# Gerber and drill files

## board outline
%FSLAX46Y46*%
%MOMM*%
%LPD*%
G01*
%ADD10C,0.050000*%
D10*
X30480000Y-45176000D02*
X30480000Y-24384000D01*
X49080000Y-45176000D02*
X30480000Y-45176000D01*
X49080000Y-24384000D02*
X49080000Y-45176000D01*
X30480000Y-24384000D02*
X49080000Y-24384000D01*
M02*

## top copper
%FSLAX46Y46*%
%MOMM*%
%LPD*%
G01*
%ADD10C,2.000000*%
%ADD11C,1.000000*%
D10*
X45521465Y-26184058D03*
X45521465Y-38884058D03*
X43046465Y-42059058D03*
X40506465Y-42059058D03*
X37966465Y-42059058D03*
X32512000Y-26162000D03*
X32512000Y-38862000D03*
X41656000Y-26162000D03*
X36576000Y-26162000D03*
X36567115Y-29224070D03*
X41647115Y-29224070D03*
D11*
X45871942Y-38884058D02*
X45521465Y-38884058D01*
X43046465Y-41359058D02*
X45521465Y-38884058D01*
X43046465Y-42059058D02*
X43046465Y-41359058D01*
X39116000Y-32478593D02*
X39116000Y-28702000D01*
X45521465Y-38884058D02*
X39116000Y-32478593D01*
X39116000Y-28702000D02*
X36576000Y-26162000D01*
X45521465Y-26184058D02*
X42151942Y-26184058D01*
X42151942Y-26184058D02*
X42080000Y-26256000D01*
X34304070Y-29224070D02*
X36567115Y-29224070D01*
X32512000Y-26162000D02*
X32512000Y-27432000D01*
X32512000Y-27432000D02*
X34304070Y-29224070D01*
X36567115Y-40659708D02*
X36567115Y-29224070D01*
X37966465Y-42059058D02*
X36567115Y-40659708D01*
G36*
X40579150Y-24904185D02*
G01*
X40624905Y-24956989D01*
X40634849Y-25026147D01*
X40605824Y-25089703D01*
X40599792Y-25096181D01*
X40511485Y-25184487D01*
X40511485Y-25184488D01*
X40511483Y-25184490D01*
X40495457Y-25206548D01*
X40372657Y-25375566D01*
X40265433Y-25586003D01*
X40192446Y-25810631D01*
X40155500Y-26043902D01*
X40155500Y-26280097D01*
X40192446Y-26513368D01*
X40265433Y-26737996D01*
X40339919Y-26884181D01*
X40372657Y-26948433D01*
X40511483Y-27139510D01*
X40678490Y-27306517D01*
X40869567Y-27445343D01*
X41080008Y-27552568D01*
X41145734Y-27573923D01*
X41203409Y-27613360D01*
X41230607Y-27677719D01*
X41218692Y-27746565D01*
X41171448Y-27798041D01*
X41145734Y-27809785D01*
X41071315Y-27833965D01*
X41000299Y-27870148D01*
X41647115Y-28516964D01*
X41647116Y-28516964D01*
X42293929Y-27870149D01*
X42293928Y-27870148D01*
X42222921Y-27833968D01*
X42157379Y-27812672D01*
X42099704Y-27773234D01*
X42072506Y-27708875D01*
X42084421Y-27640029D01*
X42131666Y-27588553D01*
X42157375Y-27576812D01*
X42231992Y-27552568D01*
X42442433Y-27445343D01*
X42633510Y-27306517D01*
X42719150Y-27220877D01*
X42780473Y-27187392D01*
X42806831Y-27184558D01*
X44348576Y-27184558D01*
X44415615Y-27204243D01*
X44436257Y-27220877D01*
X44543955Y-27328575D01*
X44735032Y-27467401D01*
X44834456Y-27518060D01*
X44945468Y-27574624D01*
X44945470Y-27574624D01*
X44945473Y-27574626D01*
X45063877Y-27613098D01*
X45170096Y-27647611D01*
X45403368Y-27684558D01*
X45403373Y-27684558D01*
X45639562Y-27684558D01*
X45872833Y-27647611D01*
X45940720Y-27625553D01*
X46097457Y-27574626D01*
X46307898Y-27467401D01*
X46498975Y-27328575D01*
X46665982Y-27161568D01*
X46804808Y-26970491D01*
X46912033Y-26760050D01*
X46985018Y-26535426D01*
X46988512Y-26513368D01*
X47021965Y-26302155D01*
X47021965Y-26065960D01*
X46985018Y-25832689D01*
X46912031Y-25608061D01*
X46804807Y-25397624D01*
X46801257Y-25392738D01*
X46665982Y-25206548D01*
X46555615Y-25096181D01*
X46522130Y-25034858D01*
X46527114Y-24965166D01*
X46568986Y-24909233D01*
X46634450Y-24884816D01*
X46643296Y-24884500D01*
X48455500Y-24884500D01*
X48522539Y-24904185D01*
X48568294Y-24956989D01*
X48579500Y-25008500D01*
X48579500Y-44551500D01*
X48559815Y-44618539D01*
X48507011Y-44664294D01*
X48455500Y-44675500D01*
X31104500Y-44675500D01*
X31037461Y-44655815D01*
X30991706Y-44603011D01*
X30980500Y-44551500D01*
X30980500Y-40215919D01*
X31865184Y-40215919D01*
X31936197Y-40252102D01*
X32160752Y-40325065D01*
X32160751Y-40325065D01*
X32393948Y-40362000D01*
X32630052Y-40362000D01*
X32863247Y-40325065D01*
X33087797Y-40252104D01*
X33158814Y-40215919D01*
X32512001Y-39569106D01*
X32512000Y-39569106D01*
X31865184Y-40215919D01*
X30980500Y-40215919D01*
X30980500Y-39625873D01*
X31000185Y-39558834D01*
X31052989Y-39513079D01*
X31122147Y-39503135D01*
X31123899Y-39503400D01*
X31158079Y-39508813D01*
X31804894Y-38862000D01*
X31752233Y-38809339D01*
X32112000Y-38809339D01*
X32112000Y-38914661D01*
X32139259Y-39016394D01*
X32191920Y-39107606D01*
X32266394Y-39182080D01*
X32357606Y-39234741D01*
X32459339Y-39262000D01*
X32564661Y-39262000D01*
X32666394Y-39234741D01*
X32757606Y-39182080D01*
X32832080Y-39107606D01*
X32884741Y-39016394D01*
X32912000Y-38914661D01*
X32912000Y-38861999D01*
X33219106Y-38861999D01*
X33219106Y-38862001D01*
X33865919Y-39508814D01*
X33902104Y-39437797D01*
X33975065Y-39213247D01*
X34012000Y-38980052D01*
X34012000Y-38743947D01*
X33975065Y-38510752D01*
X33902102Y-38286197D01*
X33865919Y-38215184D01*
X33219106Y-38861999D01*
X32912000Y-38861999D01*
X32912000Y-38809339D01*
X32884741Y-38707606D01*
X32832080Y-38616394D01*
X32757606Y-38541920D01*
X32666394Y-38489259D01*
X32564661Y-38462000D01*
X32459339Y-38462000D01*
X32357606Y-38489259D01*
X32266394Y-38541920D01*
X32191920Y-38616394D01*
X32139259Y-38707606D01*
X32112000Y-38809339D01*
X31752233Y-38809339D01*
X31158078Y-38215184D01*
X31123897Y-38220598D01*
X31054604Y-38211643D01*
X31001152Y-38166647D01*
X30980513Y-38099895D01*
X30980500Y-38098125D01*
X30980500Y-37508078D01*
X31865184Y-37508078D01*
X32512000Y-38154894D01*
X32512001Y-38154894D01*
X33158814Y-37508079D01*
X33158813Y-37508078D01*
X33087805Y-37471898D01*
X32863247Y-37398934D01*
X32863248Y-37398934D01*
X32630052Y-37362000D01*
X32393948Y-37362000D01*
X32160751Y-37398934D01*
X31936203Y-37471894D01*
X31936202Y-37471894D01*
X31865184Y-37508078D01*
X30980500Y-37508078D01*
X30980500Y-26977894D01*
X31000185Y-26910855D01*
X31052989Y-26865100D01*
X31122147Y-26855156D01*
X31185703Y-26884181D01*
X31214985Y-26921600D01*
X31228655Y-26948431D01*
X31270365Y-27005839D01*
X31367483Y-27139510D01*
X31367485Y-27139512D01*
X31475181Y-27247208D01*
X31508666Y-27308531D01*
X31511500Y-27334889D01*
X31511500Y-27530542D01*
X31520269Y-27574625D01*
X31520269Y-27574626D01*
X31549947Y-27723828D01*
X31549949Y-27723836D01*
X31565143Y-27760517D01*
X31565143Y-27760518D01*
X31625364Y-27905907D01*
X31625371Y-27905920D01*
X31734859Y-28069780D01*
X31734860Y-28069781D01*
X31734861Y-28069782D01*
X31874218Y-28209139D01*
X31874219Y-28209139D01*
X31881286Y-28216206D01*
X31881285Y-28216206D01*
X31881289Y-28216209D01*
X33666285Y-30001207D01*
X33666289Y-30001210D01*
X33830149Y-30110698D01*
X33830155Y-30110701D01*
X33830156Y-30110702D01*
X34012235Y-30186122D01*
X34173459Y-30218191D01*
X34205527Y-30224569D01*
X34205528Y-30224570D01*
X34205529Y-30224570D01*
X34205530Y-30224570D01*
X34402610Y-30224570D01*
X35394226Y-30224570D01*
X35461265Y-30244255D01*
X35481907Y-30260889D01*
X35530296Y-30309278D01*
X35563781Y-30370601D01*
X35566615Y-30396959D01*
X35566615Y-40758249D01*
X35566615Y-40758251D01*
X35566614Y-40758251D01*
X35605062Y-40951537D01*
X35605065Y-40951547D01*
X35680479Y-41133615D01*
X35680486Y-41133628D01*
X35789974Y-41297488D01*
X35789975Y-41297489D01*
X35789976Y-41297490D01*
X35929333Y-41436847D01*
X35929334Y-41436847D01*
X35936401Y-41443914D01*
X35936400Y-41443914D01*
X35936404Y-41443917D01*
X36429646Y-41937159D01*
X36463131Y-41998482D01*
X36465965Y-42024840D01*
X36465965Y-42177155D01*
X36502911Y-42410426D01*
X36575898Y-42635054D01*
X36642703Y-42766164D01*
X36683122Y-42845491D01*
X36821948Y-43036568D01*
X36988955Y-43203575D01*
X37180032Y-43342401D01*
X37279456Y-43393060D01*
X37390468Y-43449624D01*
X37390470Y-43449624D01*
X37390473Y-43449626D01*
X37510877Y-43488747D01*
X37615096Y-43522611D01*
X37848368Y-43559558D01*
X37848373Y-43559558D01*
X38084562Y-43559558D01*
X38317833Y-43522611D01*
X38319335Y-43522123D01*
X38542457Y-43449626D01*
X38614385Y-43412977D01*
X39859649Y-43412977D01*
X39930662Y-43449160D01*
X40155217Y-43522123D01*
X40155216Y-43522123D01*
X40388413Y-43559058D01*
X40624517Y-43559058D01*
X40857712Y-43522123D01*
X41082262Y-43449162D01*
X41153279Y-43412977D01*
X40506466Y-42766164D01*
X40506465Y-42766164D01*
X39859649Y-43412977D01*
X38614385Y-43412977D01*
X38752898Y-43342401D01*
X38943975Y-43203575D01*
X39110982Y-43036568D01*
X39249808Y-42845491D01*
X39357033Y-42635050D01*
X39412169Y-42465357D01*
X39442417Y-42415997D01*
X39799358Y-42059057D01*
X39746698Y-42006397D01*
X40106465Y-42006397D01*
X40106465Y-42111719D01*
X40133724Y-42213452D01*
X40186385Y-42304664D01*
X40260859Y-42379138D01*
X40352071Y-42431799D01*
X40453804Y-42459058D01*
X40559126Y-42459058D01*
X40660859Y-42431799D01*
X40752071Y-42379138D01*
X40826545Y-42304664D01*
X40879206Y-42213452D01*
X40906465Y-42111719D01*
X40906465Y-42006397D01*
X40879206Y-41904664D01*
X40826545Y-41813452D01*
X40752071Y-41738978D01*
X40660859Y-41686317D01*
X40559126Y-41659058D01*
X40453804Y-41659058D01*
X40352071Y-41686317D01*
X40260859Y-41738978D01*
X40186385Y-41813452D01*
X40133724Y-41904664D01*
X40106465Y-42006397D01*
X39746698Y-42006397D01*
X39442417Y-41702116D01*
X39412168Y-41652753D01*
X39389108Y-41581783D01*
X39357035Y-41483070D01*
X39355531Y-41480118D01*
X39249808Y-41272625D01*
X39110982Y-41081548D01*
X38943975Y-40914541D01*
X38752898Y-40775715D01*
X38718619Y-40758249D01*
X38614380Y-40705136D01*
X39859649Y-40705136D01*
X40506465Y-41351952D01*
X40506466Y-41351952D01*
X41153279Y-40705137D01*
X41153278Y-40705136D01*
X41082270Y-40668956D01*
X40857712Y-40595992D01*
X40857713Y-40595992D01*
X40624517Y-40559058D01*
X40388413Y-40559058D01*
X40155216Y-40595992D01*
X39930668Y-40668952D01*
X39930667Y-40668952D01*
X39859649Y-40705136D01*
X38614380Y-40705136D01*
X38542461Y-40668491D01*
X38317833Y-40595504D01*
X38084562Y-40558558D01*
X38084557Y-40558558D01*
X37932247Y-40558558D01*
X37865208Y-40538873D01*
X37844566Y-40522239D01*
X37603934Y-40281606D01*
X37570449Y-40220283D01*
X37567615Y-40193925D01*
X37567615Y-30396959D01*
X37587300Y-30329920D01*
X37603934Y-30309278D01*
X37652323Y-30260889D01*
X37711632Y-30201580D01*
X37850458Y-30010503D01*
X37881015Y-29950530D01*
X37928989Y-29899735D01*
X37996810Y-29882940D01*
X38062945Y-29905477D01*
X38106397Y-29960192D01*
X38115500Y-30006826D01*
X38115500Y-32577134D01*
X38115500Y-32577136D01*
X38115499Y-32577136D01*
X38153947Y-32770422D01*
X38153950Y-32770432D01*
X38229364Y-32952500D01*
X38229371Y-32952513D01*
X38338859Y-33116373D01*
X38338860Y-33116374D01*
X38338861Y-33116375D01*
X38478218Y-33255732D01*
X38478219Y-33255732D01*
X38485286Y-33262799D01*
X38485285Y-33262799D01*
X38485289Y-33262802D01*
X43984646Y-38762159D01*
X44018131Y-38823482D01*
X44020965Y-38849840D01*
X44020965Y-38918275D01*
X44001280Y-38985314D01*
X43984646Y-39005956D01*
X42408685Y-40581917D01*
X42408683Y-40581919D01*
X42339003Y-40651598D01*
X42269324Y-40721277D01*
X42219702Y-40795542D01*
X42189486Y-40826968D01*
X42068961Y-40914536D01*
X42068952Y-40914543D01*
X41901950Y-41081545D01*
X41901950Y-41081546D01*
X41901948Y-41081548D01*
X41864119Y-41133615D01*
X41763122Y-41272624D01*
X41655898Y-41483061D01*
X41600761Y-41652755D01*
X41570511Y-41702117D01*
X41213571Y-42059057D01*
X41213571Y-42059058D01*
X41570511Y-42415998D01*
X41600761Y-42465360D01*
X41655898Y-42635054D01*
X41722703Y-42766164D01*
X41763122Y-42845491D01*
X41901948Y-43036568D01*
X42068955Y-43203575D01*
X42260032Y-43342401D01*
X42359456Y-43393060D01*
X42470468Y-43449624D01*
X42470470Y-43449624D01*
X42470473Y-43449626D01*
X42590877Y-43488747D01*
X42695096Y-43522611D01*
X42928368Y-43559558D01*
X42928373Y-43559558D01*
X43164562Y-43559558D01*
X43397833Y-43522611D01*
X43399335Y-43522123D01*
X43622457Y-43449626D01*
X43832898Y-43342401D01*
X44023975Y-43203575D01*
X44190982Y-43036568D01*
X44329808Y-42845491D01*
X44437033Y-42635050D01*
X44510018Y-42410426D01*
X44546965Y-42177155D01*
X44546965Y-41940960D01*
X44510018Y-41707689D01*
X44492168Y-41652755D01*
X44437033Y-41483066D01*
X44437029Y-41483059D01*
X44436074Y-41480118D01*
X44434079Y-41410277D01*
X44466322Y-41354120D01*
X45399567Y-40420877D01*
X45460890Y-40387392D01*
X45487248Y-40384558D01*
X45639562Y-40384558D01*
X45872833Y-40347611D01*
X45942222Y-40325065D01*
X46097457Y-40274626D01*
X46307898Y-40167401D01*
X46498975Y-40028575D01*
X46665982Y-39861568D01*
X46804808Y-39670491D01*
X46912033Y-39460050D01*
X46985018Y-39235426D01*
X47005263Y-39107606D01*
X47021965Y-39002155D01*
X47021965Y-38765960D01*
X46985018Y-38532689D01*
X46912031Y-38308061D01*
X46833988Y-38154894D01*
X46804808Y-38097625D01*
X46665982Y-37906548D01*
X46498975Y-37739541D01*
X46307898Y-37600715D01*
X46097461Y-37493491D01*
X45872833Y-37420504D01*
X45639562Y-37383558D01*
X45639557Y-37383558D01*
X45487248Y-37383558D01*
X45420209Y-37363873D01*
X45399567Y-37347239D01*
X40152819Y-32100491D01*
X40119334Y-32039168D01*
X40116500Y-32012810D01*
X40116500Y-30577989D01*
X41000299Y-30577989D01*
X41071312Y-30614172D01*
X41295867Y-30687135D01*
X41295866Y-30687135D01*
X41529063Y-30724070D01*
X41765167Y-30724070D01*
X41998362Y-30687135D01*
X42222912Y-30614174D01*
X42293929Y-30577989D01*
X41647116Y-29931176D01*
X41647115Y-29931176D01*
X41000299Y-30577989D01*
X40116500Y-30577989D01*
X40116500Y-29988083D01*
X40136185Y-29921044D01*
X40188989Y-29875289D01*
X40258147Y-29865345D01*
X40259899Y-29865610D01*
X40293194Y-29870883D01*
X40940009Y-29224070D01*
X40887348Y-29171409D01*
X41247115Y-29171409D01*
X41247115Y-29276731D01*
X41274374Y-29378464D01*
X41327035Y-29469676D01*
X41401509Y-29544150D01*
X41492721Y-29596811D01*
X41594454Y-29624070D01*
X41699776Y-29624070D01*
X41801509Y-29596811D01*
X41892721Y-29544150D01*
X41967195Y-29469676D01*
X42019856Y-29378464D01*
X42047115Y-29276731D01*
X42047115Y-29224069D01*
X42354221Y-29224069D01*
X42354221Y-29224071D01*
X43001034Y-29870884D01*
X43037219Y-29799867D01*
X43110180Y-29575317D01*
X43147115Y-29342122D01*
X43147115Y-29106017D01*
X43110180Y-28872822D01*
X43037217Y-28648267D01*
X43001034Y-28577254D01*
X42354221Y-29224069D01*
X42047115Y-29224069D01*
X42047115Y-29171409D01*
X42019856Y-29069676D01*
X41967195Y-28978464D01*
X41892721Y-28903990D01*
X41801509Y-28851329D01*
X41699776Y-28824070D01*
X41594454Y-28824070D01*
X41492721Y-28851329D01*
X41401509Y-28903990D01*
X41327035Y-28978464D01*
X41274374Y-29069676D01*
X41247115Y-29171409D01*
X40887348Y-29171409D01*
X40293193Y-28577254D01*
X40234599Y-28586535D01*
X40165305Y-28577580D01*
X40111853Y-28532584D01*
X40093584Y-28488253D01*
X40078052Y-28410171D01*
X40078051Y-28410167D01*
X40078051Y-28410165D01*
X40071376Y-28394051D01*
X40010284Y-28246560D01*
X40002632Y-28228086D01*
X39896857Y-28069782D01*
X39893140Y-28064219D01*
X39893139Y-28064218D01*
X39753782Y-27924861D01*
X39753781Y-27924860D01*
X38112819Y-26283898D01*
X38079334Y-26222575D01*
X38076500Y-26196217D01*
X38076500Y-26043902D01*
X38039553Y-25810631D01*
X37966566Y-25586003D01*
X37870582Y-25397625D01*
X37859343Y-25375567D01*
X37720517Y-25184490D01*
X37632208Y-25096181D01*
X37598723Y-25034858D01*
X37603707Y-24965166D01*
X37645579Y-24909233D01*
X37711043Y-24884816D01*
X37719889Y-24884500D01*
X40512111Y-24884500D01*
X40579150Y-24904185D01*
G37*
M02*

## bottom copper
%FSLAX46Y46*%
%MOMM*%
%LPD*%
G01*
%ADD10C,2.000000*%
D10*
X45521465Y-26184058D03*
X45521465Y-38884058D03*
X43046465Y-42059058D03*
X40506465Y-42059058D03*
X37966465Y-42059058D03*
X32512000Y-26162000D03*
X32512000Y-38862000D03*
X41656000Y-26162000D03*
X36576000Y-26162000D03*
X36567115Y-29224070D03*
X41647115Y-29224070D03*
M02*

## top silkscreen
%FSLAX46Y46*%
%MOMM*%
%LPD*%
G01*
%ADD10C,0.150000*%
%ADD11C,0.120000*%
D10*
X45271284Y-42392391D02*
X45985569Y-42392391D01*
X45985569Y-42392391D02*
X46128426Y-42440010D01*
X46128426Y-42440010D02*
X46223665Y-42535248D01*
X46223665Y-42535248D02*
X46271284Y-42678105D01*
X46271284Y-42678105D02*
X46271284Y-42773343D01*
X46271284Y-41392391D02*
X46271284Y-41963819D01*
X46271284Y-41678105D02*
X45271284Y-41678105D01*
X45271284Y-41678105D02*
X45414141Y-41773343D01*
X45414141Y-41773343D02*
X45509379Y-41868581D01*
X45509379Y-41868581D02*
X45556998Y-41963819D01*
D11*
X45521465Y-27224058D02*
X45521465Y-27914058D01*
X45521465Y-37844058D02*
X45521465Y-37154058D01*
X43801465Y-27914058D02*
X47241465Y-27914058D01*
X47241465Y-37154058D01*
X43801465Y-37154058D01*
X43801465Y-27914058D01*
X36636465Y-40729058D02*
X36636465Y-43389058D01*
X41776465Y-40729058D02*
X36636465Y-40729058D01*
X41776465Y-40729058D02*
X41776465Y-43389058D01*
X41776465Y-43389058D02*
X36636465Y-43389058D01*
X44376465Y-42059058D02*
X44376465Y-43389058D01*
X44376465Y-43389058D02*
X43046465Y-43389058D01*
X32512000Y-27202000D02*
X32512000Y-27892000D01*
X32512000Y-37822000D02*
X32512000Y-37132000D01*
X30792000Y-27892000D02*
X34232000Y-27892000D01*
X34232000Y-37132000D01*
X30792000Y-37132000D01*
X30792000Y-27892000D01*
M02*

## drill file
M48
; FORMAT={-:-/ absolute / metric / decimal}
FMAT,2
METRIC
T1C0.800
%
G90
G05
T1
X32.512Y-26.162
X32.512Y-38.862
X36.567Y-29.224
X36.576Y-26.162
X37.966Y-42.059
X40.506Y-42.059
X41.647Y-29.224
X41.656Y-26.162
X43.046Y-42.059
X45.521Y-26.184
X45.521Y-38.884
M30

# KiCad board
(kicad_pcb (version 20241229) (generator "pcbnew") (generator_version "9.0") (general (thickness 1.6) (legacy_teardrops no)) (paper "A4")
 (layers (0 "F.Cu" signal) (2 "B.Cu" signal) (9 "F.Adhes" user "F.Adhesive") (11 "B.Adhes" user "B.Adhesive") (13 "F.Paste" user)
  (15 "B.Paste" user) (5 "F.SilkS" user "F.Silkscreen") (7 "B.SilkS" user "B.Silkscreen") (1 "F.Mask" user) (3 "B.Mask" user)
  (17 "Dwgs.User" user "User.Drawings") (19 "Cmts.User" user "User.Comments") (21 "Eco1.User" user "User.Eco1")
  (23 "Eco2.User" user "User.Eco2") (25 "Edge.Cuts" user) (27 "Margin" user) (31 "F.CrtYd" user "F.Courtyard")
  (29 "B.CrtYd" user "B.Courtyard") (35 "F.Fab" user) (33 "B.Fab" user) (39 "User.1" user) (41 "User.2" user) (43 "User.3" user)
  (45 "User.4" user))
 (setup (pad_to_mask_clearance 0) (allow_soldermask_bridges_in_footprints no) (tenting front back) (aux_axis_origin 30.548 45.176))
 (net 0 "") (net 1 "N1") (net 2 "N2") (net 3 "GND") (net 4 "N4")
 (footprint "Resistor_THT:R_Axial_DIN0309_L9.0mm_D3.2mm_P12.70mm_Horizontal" (layer "F.Cu") (at 45.521465 26.184058 -90)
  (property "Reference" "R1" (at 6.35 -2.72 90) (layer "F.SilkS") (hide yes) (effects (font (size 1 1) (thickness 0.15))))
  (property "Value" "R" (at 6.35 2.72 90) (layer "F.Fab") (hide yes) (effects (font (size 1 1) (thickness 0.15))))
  (fp_line (start 1.04 0) (end 1.73 0) (stroke (width 0.12) (type solid)) (layer "F.SilkS"))
  (fp_line (start 11.66 0) (end 10.97 0) (stroke (width 0.12) (type solid)) (layer "F.SilkS"))
  (fp_rect (start 1.73 -1.72) (end 10.97 1.72) (stroke (width 0.12) (type solid)) (fill no) (layer "F.SilkS"))
  (pad "1" thru_hole circle (at 0 0 270) (size 2 2) (drill 0.8) (layers "*.Cu" "*.Mask") (remove_unused_layers no) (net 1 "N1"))
  (pad "2" thru_hole circle (at 12.7 0 270) (size 2 2) (drill 0.8) (layers "*.Cu" "*.Mask") (remove_unused_layers no) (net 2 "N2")))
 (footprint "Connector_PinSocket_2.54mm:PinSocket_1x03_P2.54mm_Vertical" (layer "F.Cu") (at 43.046465 42.059058 -90)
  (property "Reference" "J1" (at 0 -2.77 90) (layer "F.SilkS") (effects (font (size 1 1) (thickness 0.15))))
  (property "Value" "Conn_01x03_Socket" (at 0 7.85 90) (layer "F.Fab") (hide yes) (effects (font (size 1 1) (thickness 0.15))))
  (fp_line (start -1.33 6.41) (end 1.33 6.41) (stroke (width 0.12) (type solid)) (layer "F.SilkS"))
  (fp_line (start -1.33 1.27) (end -1.33 6.41) (stroke (width 0.12) (type solid)) (layer "F.SilkS"))
  (fp_line (start -1.33 1.27) (end 1.33 1.27) (stroke (width 0.12) (type solid)) (layer "F.SilkS"))
  (fp_line (start 1.33 1.27) (end 1.33 6.41) (stroke (width 0.12) (type solid)) (layer "F.SilkS"))
  (fp_line (start 0 -1.33) (end 1.33 -1.33) (stroke (width 0.12) (type solid)) (layer "F.SilkS"))
  (fp_line (start 1.33 -1.33) (end 1.33 0) (stroke (width 0.12) (type solid)) (layer "F.SilkS"))
  (pad "1" thru_hole circle (at 0 0 270) (size 2 2) (drill 0.8) (layers "*.Cu" "*.Mask") (remove_unused_layers no) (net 2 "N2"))
  (pad "2" thru_hole circle (at 0 2.54 270) (size 2 2) (drill 0.8) (layers "*.Cu" "*.Mask") (remove_unused_layers no) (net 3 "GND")
   (thermal_bridge_width 1))
  (pad "3" thru_hole circle (at 0 5.08 270) (size 2 2) (drill 0.8) (layers "*.Cu" "*.Mask") (remove_unused_layers no) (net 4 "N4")))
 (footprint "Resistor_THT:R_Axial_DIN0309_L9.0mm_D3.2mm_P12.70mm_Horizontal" (layer "F.Cu") (at 32.512 26.162 -90)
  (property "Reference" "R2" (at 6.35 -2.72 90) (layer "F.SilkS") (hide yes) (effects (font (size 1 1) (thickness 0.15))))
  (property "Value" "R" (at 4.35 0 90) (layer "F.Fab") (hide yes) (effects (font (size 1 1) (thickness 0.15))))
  (fp_line (start 1.04 0) (end 1.73 0) (stroke (width 0.12) (type solid)) (layer "F.SilkS"))
  (fp_line (start 11.66 0) (end 10.97 0) (stroke (width 0.12) (type solid)) (layer "F.SilkS"))
  (fp_rect (start 1.73 -1.72) (end 10.97 1.72) (stroke (width 0.12) (type solid)) (fill no) (layer "F.SilkS"))
  (pad "1" thru_hole circle (at 0 0 270) (size 2 2) (drill 0.8) (layers "*.Cu" "*.Mask") (remove_unused_layers no) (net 4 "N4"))
  (pad "2" thru_hole circle (at 12.7 0 270) (size 2 2) (drill 0.8) (layers "*.Cu" "*.Mask") (remove_unused_layers no) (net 3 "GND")
   (thermal_bridge_width 1)))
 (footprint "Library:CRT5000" (layer "F.Cu") (at 39.107115 29.22407 -90)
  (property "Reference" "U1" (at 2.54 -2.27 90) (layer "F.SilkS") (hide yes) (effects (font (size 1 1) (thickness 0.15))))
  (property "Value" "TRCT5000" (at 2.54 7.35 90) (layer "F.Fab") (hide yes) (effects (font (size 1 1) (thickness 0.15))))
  (pad "1" thru_hole circle (at -3.06207 -2.548885 270) (size 2 2) (drill 0.8) (layers "*.Cu" "*.Mask") (remove_unused_layers no)
   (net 1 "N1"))
  (pad "2" thru_hole circle (at -3.06207 2.531115 270) (size 2 2) (drill 0.8) (layers "*.Cu" "*.Mask") (remove_unused_layers no)
   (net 2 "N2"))
  (pad "3" thru_hole circle (at 0 2.54 270) (size 2 2) (drill 0.8) (layers "*.Cu" "*.Mask") (remove_unused_layers no) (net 4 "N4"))
  (pad "4" thru_hole circle (at 0 -2.54 270) (size 2 2) (drill 0.8) (layers "*.Cu" "*.Mask") (remove_unused_layers no) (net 3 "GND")
   (thermal_bridge_width 1)))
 (gr_line (start 30.48 45.176) (end 30.48 24.384) (stroke (width 0.05) (type default)) (layer "Edge.Cuts"))
 (gr_line (start 49.08 45.176) (end 30.48 45.176) (stroke (width 0.05) (type default)) (layer "Edge.Cuts"))
 (gr_line (start 49.08 24.384) (end 49.08 45.176) (stroke (width 0.05) (type default)) (layer "Edge.Cuts"))
 (gr_line (start 30.48 24.384) (end 49.08 24.384) (stroke (width 0.05) (type default)) (layer "Edge.Cuts"))
 (segment (start 45.871942 38.884058) (end 45.521465 38.884058) (width 1) (layer "F.Cu") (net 2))
 (segment (start 43.046465 41.359058) (end 45.521465 38.884058) (width 1) (layer "F.Cu") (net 2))
 (segment (start 43.046465 42.059058) (end 43.046465 41.359058) (width 1) (layer "F.Cu") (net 2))
 (segment (start 39.116 32.478593) (end 39.116 28.702) (width 1) (layer "F.Cu") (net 2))
 (segment (start 45.521465 38.884058) (end 39.116 32.478593) (width 1) (layer "F.Cu") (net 2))
 (segment (start 39.116 28.702) (end 36.576 26.162) (width 1) (layer "F.Cu") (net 2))
 (segment (start 45.521465 26.184058) (end 42.151942 26.184058) (width 1) (layer "F.Cu") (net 1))
 (segment (start 42.151942 26.184058) (end 42.08 26.256) (width 1) (layer "F.Cu") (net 1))
 (segment (start 34.30407 29.22407) (end 36.567115 29.22407) (width 1) (layer "F.Cu") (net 4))
 (segment (start 32.512 26.162) (end 32.512 27.432) (width 1) (layer "F.Cu") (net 4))
 (segment (start 32.512 27.432) (end 34.30407 29.22407) (width 1) (layer "F.Cu") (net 4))
 (segment (start 36.567115 40.659708) (end 36.567115 29.22407) (width 1) (layer "F.Cu") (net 4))
 (segment (start 37.966465 42.059058) (end 36.567115 40.659708) (width 1) (layer "F.Cu") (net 4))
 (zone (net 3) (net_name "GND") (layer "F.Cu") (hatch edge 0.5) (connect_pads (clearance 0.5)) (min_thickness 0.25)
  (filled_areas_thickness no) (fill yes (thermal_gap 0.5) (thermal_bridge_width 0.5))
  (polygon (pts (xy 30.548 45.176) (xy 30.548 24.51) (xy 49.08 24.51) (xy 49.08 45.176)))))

